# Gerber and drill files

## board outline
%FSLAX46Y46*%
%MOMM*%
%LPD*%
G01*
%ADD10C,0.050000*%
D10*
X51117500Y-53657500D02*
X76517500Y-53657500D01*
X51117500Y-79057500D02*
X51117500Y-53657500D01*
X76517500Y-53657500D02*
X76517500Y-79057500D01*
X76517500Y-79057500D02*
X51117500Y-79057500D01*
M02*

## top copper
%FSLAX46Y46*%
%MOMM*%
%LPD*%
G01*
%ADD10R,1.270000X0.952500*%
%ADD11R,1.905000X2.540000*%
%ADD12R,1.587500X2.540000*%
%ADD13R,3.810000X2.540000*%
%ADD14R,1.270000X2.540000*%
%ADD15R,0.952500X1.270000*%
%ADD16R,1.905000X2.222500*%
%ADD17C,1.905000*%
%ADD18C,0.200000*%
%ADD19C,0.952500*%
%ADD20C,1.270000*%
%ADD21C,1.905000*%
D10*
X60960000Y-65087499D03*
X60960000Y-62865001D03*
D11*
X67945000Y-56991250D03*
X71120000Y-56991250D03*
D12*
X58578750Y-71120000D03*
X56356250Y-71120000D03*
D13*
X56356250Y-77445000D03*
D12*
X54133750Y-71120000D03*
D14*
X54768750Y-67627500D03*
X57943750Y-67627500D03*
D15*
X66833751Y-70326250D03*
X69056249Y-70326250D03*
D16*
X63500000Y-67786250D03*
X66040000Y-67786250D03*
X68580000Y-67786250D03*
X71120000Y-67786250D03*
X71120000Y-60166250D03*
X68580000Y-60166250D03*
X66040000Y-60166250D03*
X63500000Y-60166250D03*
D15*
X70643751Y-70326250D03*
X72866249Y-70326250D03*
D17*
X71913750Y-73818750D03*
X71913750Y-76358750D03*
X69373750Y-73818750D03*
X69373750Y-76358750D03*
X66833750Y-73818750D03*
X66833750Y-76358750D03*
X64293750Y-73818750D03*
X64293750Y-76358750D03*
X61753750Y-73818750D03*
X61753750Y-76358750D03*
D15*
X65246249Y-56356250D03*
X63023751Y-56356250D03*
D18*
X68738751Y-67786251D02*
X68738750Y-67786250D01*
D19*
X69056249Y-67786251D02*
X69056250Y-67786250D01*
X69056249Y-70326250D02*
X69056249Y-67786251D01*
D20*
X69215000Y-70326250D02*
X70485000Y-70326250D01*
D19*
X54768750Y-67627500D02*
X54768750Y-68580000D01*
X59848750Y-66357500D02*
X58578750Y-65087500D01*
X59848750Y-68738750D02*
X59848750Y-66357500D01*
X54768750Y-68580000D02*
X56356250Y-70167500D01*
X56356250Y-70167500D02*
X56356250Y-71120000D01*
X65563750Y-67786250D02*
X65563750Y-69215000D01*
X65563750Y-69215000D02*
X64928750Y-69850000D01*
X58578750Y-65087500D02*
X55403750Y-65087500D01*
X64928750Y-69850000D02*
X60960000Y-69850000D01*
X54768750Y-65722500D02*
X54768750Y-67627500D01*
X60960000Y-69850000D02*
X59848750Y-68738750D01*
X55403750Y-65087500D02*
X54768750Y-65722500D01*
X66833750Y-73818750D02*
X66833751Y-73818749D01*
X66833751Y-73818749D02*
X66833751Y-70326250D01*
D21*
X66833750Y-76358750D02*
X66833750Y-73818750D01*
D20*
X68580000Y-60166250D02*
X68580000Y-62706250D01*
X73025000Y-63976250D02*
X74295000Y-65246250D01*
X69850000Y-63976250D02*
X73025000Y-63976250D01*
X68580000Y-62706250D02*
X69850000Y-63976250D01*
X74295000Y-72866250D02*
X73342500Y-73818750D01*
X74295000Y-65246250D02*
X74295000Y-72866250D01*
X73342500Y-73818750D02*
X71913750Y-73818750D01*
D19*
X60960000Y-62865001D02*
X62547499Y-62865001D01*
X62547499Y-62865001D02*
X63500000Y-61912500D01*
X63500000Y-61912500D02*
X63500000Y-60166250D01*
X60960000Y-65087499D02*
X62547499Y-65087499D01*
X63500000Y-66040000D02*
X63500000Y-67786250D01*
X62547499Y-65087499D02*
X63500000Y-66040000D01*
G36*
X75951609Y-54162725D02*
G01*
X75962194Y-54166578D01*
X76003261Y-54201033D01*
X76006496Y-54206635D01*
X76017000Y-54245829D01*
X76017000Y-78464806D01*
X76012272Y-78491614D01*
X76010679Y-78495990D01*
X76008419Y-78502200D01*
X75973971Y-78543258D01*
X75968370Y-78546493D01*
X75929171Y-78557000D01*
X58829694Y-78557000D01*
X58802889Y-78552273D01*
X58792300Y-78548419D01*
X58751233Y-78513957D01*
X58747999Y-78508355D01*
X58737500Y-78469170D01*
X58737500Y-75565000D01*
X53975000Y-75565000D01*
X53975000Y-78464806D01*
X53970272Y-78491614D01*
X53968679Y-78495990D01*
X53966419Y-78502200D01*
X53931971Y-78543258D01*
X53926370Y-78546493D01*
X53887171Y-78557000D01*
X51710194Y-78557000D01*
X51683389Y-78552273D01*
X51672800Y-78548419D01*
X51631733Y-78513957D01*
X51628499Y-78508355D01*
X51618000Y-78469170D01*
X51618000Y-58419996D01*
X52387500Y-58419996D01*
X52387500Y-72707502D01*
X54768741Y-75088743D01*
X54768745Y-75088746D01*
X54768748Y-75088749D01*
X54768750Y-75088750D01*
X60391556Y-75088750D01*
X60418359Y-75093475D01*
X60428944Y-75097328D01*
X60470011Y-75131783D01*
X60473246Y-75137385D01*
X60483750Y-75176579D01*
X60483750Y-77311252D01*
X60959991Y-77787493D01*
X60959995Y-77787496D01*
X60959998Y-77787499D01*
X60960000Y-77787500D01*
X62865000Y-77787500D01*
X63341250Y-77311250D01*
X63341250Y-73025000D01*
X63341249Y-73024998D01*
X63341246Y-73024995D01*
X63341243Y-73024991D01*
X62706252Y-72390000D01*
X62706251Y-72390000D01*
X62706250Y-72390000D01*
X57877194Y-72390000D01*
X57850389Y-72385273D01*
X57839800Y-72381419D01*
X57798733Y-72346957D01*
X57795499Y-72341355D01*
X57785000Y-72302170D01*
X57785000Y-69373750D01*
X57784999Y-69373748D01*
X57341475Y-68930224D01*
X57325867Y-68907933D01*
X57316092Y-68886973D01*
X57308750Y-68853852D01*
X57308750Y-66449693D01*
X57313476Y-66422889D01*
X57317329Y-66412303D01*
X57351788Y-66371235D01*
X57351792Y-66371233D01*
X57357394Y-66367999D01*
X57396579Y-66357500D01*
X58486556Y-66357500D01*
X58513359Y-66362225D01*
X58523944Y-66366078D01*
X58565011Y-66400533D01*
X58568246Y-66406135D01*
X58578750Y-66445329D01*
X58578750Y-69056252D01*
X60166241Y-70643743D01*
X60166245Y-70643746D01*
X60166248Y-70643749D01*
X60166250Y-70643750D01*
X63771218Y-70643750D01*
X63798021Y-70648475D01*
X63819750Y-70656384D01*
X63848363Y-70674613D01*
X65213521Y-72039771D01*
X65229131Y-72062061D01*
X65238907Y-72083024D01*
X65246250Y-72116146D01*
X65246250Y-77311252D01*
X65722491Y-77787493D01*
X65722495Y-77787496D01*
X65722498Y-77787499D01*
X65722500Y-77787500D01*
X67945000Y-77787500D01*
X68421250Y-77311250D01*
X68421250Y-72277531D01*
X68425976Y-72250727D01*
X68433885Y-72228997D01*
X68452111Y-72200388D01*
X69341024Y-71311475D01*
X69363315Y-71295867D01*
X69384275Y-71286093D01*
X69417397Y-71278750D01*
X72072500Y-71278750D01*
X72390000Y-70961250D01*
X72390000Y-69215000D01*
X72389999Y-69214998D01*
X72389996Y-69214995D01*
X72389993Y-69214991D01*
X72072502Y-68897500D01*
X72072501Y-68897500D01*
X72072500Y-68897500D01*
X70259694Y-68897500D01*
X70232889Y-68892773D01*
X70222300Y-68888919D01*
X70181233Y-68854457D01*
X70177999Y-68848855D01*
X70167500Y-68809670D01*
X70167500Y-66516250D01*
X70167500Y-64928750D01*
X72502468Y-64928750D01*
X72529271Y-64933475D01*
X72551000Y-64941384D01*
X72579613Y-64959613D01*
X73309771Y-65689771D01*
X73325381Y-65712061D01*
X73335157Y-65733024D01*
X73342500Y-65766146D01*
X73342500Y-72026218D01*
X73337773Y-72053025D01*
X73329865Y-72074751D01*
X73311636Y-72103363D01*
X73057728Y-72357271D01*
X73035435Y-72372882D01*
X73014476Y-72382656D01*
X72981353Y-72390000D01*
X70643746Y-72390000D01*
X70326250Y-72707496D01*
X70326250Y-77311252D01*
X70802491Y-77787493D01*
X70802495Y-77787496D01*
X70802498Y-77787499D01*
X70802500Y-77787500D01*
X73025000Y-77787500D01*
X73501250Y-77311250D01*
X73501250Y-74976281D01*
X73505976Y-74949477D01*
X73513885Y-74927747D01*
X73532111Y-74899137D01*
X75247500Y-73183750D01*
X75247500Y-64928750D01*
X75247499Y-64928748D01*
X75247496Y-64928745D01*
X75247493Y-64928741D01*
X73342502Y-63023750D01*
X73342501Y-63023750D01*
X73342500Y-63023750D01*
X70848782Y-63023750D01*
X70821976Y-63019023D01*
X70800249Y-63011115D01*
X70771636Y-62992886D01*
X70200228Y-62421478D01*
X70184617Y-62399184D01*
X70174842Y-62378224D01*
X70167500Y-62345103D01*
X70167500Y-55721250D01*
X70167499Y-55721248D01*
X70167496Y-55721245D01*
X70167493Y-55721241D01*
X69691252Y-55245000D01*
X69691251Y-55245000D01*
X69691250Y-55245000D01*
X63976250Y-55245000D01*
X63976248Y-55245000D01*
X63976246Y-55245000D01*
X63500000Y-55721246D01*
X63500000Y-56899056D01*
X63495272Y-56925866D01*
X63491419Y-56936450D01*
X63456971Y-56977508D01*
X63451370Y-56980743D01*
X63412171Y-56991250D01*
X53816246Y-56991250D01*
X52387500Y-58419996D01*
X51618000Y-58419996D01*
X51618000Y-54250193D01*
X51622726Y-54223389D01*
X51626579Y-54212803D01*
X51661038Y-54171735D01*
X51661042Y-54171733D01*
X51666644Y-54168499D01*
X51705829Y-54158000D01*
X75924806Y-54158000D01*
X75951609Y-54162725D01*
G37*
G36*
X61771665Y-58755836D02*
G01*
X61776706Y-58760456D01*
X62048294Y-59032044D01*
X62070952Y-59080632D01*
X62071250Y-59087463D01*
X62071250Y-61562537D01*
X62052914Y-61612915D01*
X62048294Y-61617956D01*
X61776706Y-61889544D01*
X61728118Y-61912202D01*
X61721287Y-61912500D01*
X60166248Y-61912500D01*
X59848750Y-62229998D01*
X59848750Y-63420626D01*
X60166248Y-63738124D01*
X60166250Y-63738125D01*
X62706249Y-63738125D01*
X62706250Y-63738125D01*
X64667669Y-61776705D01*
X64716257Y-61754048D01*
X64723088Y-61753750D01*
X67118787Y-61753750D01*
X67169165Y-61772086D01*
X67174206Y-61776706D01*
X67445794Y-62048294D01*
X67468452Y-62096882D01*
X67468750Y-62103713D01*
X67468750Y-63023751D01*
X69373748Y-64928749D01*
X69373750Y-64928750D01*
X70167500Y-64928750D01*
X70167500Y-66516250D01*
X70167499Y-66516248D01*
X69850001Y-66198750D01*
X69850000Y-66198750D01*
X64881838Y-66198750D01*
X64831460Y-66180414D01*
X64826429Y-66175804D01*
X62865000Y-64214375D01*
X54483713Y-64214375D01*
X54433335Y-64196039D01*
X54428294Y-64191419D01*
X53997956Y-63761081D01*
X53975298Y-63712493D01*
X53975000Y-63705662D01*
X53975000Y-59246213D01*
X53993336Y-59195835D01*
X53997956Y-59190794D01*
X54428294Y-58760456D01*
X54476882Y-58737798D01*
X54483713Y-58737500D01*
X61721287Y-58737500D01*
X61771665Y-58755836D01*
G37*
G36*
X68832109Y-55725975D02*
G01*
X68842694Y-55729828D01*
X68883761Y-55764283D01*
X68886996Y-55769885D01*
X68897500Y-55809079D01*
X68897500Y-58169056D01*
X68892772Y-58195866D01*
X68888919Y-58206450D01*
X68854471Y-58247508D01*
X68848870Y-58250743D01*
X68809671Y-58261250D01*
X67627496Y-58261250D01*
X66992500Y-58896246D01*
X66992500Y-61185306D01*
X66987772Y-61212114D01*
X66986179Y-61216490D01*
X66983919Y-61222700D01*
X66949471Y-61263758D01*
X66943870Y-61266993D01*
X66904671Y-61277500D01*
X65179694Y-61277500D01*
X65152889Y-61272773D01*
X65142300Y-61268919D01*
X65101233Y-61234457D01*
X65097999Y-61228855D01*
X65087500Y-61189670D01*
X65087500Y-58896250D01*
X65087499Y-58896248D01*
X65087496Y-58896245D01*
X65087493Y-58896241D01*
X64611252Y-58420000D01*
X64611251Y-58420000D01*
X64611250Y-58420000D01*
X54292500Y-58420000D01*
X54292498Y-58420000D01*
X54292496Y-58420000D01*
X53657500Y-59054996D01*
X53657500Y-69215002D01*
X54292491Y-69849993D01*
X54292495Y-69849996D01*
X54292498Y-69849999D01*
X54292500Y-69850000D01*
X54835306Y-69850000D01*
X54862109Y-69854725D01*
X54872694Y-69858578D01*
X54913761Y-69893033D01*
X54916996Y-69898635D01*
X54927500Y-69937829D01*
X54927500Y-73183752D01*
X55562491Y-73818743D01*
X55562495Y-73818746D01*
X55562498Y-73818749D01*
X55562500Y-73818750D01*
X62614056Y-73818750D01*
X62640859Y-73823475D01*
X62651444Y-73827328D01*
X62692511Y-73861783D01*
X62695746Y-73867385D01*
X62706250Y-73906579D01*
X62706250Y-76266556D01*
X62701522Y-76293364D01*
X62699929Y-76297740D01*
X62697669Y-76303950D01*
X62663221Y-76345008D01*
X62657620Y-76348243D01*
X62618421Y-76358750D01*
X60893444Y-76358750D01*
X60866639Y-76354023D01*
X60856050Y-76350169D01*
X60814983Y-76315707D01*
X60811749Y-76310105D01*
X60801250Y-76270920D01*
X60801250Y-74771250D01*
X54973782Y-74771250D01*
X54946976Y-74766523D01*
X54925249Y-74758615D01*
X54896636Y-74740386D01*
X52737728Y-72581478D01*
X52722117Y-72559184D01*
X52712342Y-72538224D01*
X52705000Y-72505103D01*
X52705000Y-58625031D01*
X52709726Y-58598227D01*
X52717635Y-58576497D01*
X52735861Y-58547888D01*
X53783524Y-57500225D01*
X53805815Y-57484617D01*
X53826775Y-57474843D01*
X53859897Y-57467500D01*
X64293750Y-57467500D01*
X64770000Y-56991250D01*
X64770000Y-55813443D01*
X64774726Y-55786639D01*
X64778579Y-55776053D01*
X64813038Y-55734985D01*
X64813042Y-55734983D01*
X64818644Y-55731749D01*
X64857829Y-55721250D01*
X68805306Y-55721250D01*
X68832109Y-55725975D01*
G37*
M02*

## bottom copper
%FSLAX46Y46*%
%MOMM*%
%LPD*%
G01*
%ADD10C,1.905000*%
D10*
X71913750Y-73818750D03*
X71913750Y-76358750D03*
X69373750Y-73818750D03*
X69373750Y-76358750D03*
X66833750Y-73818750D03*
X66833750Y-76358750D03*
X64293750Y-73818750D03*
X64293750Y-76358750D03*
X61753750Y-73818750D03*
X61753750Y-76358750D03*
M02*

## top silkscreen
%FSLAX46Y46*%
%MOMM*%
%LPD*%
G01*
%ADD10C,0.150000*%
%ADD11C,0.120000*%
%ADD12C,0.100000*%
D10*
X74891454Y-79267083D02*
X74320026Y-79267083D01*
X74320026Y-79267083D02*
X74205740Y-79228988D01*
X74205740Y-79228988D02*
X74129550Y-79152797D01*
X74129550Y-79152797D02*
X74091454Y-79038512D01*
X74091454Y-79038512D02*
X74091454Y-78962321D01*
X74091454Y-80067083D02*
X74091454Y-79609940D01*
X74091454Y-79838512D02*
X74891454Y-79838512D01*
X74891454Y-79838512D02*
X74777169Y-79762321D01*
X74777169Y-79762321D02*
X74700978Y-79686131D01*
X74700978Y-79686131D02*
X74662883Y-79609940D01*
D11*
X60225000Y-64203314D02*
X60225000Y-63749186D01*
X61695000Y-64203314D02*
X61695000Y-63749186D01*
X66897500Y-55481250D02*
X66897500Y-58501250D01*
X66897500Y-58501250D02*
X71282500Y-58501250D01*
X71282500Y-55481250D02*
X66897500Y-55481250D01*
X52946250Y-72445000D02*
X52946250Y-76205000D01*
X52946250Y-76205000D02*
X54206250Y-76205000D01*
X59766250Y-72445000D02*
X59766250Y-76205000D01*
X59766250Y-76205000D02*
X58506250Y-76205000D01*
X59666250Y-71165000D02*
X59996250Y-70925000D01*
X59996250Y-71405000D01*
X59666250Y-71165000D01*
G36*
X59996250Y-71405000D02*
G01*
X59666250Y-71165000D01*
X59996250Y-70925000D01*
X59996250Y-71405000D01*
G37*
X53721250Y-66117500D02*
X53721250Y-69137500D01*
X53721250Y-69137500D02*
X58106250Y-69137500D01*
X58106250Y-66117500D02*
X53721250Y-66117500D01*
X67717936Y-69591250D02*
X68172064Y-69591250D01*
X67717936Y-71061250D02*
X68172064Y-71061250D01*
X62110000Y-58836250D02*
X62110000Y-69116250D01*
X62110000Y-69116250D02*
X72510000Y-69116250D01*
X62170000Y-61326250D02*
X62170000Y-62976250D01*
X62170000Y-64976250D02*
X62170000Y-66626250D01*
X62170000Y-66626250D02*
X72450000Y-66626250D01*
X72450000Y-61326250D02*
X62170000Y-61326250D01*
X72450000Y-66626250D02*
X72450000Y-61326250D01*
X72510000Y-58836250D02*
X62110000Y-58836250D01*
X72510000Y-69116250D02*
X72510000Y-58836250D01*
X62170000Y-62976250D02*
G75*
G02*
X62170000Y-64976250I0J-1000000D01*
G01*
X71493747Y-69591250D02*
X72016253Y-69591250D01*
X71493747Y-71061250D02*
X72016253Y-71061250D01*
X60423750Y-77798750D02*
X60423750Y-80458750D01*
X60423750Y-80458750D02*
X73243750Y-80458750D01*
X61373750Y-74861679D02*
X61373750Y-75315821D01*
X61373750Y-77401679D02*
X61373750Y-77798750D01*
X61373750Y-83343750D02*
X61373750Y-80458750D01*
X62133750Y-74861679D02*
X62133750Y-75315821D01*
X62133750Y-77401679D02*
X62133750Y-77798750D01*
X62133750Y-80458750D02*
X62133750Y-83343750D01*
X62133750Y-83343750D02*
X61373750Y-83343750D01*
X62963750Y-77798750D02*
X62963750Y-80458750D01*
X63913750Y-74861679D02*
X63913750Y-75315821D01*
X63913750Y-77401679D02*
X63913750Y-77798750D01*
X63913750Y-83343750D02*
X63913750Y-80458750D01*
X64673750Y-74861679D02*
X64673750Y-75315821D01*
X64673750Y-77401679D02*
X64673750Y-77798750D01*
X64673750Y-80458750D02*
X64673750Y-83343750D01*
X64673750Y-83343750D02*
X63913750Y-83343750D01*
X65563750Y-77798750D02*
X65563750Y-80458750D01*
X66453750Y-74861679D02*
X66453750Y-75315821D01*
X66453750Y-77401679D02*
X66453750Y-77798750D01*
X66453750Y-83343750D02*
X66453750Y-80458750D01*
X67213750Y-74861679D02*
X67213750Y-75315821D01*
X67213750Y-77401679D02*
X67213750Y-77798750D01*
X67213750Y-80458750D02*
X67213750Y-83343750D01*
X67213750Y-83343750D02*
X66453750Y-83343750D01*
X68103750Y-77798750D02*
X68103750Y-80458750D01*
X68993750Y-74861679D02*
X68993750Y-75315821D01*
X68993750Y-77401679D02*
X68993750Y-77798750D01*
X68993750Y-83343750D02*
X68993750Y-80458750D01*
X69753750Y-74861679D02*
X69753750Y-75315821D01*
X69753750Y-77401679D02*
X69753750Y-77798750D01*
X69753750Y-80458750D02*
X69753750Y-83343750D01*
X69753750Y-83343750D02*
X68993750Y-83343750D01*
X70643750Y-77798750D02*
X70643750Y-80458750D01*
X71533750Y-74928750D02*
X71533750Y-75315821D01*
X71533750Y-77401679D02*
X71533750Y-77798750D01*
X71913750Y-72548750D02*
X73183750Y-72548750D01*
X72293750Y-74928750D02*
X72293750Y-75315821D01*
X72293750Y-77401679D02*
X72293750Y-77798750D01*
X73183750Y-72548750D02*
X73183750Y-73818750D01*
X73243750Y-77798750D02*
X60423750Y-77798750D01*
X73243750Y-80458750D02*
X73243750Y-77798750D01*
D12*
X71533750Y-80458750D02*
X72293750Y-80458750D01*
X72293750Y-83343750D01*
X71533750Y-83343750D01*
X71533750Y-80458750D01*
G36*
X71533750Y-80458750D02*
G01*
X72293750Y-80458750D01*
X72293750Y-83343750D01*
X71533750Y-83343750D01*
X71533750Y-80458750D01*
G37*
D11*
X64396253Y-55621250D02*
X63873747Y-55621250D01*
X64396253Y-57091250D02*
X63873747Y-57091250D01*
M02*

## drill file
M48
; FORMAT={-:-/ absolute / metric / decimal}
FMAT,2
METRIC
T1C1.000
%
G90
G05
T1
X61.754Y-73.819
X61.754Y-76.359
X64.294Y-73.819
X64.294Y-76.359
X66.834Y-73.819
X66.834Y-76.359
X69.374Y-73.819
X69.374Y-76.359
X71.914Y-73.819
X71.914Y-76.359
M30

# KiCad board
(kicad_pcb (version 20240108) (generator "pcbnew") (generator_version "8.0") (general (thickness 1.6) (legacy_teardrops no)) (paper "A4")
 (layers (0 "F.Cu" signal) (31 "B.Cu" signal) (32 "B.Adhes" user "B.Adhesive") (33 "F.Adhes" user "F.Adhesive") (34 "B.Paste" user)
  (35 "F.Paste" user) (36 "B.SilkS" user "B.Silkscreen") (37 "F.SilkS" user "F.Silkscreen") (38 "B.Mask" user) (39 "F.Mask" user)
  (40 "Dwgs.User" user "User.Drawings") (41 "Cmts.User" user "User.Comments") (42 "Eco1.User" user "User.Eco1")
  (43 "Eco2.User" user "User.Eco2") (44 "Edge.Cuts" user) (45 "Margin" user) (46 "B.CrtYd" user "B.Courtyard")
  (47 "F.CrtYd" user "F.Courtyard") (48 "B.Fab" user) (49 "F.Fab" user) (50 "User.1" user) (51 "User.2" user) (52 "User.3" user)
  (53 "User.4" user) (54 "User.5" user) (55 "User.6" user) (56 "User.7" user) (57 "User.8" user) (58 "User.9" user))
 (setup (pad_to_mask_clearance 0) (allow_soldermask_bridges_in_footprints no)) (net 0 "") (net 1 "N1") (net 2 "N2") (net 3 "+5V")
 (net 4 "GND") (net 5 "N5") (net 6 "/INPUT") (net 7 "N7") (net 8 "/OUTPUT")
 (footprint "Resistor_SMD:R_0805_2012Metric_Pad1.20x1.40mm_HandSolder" (layer "F.Cu") (at 60.96 63.97625 90)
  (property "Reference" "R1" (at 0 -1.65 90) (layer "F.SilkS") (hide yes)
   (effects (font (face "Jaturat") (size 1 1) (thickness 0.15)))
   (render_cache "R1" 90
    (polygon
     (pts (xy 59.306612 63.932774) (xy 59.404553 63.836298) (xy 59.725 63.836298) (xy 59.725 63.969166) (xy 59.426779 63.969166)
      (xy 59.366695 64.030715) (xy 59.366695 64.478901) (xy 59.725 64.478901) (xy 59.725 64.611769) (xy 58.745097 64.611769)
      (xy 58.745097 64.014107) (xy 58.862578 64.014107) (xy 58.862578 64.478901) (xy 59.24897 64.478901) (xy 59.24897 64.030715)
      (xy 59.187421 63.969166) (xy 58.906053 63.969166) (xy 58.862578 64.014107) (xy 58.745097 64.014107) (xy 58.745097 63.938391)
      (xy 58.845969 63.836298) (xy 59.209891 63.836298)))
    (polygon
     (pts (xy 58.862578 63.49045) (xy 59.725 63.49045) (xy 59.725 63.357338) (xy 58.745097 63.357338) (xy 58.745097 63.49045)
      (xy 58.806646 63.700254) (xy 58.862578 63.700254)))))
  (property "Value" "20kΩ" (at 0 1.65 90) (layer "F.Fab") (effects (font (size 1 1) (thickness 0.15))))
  (fp_line (start -0.227064 -0.735) (end 0.227064 -0.735) (stroke (width 0.12) (type solid)) (layer "F.SilkS"))
  (fp_line (start -0.227064 0.735) (end 0.227064 0.735) (stroke (width 0.12) (type solid)) (layer "F.SilkS"))
  (pad "1" smd rect (at -1.111249 0 90) (size 0.9525 1.27) (layers "F.Cu" "F.Paste" "F.Mask") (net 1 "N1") (clearance 0.15875))
  (pad "2" smd rect (at 1.111249 0 90) (size 0.9525 1.27) (layers "F.Cu" "F.Paste" "F.Mask") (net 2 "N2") (clearance 0.15875)))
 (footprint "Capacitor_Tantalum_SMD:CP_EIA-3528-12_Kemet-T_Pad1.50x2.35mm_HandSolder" (layer "F.Cu") (at 69.5325 56.99125)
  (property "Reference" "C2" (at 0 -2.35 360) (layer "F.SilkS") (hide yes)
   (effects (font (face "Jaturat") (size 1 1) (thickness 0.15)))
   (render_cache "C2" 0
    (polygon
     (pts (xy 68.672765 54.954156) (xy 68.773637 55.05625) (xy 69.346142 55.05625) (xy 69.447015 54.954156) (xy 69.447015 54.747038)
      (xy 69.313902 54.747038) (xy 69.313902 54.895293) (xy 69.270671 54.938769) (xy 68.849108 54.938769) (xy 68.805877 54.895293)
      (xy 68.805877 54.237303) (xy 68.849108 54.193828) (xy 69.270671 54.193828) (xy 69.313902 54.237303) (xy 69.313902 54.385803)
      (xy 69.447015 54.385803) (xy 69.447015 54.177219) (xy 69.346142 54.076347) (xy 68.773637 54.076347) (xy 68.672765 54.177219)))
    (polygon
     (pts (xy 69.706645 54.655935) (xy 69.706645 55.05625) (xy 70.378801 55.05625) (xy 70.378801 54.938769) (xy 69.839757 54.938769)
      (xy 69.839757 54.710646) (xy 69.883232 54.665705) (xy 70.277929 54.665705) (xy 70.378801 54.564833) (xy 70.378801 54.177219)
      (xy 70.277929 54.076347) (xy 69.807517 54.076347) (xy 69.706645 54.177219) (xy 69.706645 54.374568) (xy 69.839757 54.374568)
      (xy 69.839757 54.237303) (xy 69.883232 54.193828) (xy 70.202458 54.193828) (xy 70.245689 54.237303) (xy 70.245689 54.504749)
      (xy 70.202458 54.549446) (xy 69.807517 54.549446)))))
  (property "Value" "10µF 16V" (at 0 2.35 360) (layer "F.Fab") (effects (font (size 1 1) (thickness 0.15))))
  (fp_line (start -2.635 -1.51) (end -2.635 1.51) (stroke (width 0.12) (type solid)) (layer "F.SilkS"))
  (fp_line (start -2.635 1.51) (end 1.75 1.51) (stroke (width 0.12) (type solid)) (layer "F.SilkS"))
  (fp_line (start 1.75 -1.51) (end -2.635 -1.51) (stroke (width 0.12) (type solid)) (layer "F.SilkS"))
  (pad "1" smd rect (at -1.5875 0) (size 1.905 2.54) (layers "F.Cu" "F.Paste" "F.Mask") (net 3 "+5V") (clearance 0.15875))
  (pad "2" smd rect (at 1.5875 0) (size 1.905 2.54) (layers "F.Cu" "F.Paste" "F.Mask") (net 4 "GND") (clearance 0.15875)))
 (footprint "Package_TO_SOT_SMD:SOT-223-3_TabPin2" (layer "F.Cu") (at 56.35625 74.295 -90)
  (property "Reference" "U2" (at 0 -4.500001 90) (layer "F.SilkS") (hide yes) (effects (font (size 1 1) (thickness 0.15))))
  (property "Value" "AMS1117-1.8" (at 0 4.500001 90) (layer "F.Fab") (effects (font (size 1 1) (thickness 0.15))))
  (fp_line (start -1.85 3.41) (end 1.91 3.41) (stroke (width 0.12) (type solid)) (layer "F.SilkS"))
  (fp_line (start 1.91 3.41) (end 1.91 2.15) (stroke (width 0.12) (type solid)) (layer "F.SilkS"))
  (fp_line (start -1.85 -3.41) (end 1.91 -3.41) (stroke (width 0.12) (type solid)) (layer "F.SilkS"))
  (fp_line (start 1.91 -3.41) (end 1.91 -2.15) (stroke (width 0.12) (type solid)) (layer "F.SilkS"))
  (fp_poly
   (pts (xy -3.13 -3.31) (xy -3.37 -3.64) (xy -2.89 -3.64) (xy -3.13 -3.31)) (stroke (width 0.12) (type solid)) (fill solid)
   (layer "F.SilkS"))
  (pad "1" smd rect (at -3.175 -2.2225 270) (size 2.54 1.5875) (layers "F.Cu" "F.Paste" "F.Mask") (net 4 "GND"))
  (pad "2" smd rect (at -3.175 0 270) (size 2.54 1.5875) (layers "F.Cu" "F.Paste" "F.Mask") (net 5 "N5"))
  (pad "2" smd rect (at 3.15 0 270) (size 2.54 3.81) (layers "F.Cu" "F.Paste" "F.Mask") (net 5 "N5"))
  (pad "3" smd rect (at -3.175 2.2225 270) (size 2.54 1.5875) (layers "F.Cu" "F.Paste" "F.Mask") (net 3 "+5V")))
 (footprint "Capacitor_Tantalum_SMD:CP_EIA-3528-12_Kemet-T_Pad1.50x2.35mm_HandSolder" (layer "F.Cu") (at 56.35625 67.6275)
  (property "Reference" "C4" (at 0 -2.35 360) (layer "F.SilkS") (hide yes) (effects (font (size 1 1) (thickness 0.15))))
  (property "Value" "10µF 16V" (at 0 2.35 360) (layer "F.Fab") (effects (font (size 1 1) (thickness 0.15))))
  (fp_line (start -2.635 -1.51) (end -2.635 1.51) (stroke (width 0.12) (type solid)) (layer "F.SilkS"))
  (fp_line (start -2.635 1.51) (end 1.75 1.51) (stroke (width 0.12) (type solid)) (layer "F.SilkS"))
  (fp_line (start 1.75 -1.51) (end -2.635 -1.51) (stroke (width 0.12) (type solid)) (layer "F.SilkS"))
  (pad "1" smd rect (at -1.5875 0) (size 1.27 2.54) (layers "F.Cu" "F.Paste" "F.Mask") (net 5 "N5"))
  (pad "2" smd rect (at 1.5875 0) (size 1.27 2.54) (layers "F.Cu" "F.Paste" "F.Mask") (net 4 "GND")))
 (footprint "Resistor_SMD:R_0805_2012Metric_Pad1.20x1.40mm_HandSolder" (layer "F.Cu") (at 67.945 70.32625)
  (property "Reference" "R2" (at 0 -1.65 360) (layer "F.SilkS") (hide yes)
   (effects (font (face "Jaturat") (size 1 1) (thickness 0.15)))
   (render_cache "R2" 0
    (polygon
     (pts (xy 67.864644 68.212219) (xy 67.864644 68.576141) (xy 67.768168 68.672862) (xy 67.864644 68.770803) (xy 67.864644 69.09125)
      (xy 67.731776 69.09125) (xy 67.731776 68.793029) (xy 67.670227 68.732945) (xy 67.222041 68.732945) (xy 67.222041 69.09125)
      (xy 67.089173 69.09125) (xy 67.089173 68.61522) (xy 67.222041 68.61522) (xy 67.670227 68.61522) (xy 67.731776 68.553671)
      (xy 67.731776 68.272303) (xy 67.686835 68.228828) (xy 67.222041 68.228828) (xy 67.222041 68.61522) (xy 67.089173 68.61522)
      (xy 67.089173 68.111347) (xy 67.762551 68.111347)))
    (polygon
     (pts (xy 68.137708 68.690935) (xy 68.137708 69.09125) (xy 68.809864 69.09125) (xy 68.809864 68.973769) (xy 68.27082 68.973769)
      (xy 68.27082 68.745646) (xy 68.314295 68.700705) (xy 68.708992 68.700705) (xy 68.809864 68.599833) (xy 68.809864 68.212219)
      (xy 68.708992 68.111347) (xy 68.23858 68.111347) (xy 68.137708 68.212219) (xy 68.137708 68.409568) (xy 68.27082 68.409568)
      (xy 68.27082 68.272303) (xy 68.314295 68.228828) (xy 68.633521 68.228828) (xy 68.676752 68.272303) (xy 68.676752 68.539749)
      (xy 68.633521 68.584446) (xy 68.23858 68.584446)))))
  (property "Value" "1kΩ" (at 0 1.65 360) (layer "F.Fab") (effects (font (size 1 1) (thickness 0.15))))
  (fp_line (start -0.227064 -0.735) (end 0.227064 -0.735) (stroke (width 0.12) (type solid)) (layer "F.SilkS"))
  (fp_line (start -0.227064 0.735) (end 0.227064 0.735) (stroke (width 0.12) (type solid)) (layer "F.SilkS"))
  (pad "1" smd rect (at -1.111249 0) (size 0.9525 1.27) (layers "F.Cu" "F.Paste" "F.Mask") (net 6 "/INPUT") (clearance 0.15875))
  (pad "2" smd rect (at 1.111249 0) (size 0.9525 1.27) (layers "F.Cu" "F.Paste" "F.Mask") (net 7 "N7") (clearance 0.15875)))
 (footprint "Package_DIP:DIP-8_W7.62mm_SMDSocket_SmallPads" (layer "F.Cu") (at 67.31 63.97625 90)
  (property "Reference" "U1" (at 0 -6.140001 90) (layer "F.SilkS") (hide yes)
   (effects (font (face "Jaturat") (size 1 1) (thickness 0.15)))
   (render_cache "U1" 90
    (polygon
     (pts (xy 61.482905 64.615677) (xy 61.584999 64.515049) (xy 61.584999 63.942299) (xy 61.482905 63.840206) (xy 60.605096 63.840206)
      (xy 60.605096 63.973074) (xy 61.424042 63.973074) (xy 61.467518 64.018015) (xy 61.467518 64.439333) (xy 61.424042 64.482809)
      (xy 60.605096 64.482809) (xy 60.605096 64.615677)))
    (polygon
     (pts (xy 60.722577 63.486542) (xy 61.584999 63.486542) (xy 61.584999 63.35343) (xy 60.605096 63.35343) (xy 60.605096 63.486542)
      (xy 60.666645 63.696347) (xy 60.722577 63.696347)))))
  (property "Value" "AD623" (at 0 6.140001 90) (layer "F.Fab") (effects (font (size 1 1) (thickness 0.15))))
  (fp_line (start 5.14 -5.2) (end -5.14 -5.2) (stroke (width 0.12) (type solid)) (layer "F.SilkS"))
  (fp_line (start -5.14 -5.2) (end -5.14 5.2) (stroke (width 0.12) (type solid)) (layer "F.SilkS"))
  (fp_line (start 2.65 -5.14) (end 1 -5.14) (stroke (width 0.12) (type solid)) (layer "F.SilkS"))
  (fp_line (start -1 -5.14) (end -2.65 -5.14) (stroke (width 0.12) (type solid)) (layer "F.SilkS"))
  (fp_line (start -2.65 -5.14) (end -2.65 5.14) (stroke (width 0.12) (type solid)) (layer "F.SilkS"))
  (fp_line (start 2.65 5.14) (end 2.65 -5.14) (stroke (width 0.12) (type solid)) (layer "F.SilkS"))
  (fp_line (start -2.65 5.14) (end 2.65 5.14) (stroke (width 0.12) (type solid)) (layer "F.SilkS"))
  (fp_line (start 5.14 5.2) (end 5.14 -5.2) (stroke (width 0.12) (type solid)) (layer "F.SilkS"))
  (fp_line (start -5.14 5.2) (end 5.14 5.2) (stroke (width 0.12) (type solid)) (layer "F.SilkS"))
  (fp_arc (start 1 -5.14) (mid 0 -4.14) (end -1 -5.14) (stroke (width 0.12) (type solid)) (layer "F.SilkS"))
  (pad "1" smd rect (at -3.81 -3.81 90) (size 2.2225 1.905) (layers "F.Cu" "F.Paste" "F.Mask") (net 1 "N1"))
  (pad "2" smd rect (at -3.81 -1.27 90) (size 2.2225 1.905) (layers "F.Cu" "F.Paste" "F.Mask") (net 5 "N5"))
  (pad "3" smd rect (at -3.81 1.27 90) (size 2.2225 1.905) (layers "F.Cu" "F.Paste" "F.Mask") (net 7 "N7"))
  (pad "4" smd rect (at -3.81 3.81 90) (size 2.2225 1.905) (layers "F.Cu" "F.Paste" "F.Mask") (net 4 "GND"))
  (pad "5" smd rect (at 3.81 3.81 90) (size 2.2225 1.905) (layers "F.Cu" "F.Paste" "F.Mask") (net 4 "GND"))
  (pad "6" smd rect (at 3.81 1.27 90) (size 2.2225 1.905) (layers "F.Cu" "F.Paste" "F.Mask") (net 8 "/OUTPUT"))
  (pad "7" smd rect (at 3.81 -1.27 90) (size 2.2225 1.905) (layers "F.Cu" "F.Paste" "F.Mask") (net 3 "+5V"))
  (pad "8" smd rect (at 3.81 -3.81 90) (size 2.2225 1.905) (layers "F.Cu" "F.Paste" "F.Mask") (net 2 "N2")))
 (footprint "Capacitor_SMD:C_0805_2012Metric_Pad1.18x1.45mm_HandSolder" (layer "F.Cu") (at 71.755 70.32625)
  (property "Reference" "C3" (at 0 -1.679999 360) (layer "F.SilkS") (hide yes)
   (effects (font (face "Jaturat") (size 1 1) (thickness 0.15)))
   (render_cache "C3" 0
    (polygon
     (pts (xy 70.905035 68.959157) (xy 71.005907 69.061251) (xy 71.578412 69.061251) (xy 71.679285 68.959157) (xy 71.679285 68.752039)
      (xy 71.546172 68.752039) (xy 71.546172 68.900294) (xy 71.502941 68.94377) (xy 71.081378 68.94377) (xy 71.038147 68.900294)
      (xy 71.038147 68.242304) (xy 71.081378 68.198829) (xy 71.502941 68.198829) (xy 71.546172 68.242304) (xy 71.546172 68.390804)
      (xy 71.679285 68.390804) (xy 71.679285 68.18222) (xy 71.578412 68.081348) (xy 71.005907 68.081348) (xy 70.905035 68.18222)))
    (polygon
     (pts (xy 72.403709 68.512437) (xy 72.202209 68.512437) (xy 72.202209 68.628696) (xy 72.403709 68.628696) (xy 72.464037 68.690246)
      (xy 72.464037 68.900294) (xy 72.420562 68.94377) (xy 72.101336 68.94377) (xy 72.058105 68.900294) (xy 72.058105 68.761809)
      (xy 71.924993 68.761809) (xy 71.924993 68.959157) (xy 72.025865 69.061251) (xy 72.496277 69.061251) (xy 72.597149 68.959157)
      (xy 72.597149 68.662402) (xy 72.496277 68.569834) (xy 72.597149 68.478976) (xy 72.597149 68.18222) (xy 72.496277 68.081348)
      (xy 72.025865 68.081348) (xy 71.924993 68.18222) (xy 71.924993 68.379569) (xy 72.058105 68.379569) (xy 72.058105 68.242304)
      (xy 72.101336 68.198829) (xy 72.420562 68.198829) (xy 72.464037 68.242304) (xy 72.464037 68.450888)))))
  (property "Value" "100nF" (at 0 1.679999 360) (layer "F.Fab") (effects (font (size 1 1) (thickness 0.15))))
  (fp_line (start -0.261253 -0.735) (end 0.261253 -0.735) (stroke (width 0.12) (type solid)) (layer "F.SilkS"))
  (fp_line (start -0.261253 0.735) (end 0.261253 0.735) (stroke (width 0.12) (type solid)) (layer "F.SilkS"))
  (pad "1" smd rect (at -1.111249 0) (size 0.9525 1.27) (layers "F.Cu" "F.Paste" "F.Mask") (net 7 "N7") (clearance 0.15875))
  (pad "2" smd rect (at 1.111249 0) (size 0.9525 1.27) (layers "F.Cu" "F.Paste" "F.Mask") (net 4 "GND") (clearance 0.15875)))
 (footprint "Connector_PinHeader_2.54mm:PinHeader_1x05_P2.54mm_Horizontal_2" (layer "F.Cu") (at 71.91375 73.81875 -90)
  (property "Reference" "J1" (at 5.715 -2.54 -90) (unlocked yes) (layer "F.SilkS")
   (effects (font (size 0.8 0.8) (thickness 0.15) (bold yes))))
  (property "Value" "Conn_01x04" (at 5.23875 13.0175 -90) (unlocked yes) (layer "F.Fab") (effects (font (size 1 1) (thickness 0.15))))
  (fp_line (start 3.98 11.49) (end 6.64 11.49) (stroke (width 0.12) (type solid)) (layer "F.SilkS"))
  (fp_line (start 6.64 11.49) (end 6.64 -1.33) (stroke (width 0.12) (type solid)) (layer "F.SilkS"))
  (fp_line (start 1.042929 10.54) (end 1.497071 10.54) (stroke (width 0.12) (type solid)) (layer "F.SilkS"))
  (fp_line (start 3.582929 10.54) (end 3.98 10.54) (stroke (width 0.12) (type solid)) (layer "F.SilkS"))
  (fp_line (start 9.525 10.54) (end 6.64 10.54) (stroke (width 0.12) (type solid)) (layer "F.SilkS"))
  (fp_line (start 1.042929 9.78) (end 1.497071 9.78) (stroke (width 0.12) (type solid)) (layer "F.SilkS"))
  (fp_line (start 3.582929 9.78) (end 3.98 9.78) (stroke (width 0.12) (type solid)) (layer "F.SilkS"))
  (fp_line (start 6.64 9.78) (end 9.525 9.78) (stroke (width 0.12) (type solid)) (layer "F.SilkS"))
  (fp_line (start 9.525 9.78) (end 9.525 10.54) (stroke (width 0.12) (type solid)) (layer "F.SilkS"))
  (fp_line (start 3.98 8.95) (end 6.64 8.95) (stroke (width 0.12) (type solid)) (layer "F.SilkS"))
  (fp_line (start 1.042929 8) (end 1.497071 8) (stroke (width 0.12) (type solid)) (layer "F.SilkS"))
  (fp_line (start 3.582929 8) (end 3.98 8) (stroke (width 0.12) (type solid)) (layer "F.SilkS"))
  (fp_line (start 9.525 8) (end 6.64 8) (stroke (width 0.12) (type solid)) (layer "F.SilkS"))
  (fp_line (start 1.042929 7.24) (end 1.497071 7.24) (stroke (width 0.12) (type solid)) (layer "F.SilkS"))
  (fp_line (start 3.582929 7.24) (end 3.98 7.24) (stroke (width 0.12) (type solid)) (layer "F.SilkS"))
  (fp_line (start 6.64 7.24) (end 9.525 7.24) (stroke (width 0.12) (type solid)) (layer "F.SilkS"))
  (fp_line (start 9.525 7.24) (end 9.525 8) (stroke (width 0.12) (type solid)) (layer "F.SilkS"))
  (fp_line (start 3.98 6.35) (end 6.64 6.35) (stroke (width 0.12) (type solid)) (layer "F.SilkS"))
  (fp_line (start 1.042929 5.46) (end 1.497071 5.46) (stroke (width 0.12) (type solid)) (layer "F.SilkS"))
  (fp_line (start 3.582929 5.46) (end 3.98 5.46) (stroke (width 0.12) (type solid)) (layer "F.SilkS"))
  (fp_line (start 9.525 5.46) (end 6.64 5.46) (stroke (width 0.12) (type solid)) (layer "F.SilkS"))
  (fp_line (start 1.042929 4.7) (end 1.497071 4.7) (stroke (width 0.12) (type solid)) (layer "F.SilkS"))
  (fp_line (start 3.582929 4.7) (end 3.98 4.7) (stroke (width 0.12) (type solid)) (layer "F.SilkS"))
  (fp_line (start 6.64 4.7) (end 9.525 4.7) (stroke (width 0.12) (type solid)) (layer "F.SilkS"))
  (fp_line (start 9.525 4.7) (end 9.525 5.46) (stroke (width 0.12) (type solid)) (layer "F.SilkS"))
  (fp_line (start 3.98 3.81) (end 6.64 3.81) (stroke (width 0.12) (type solid)) (layer "F.SilkS"))
  (fp_line (start 1.042929 2.92) (end 1.497071 2.92) (stroke (width 0.12) (type solid)) (layer "F.SilkS"))
  (fp_line (start 3.582929 2.92) (end 3.98 2.92) (stroke (width 0.12) (type solid)) (layer "F.SilkS"))
  (fp_line (start 9.525 2.92) (end 6.64 2.92) (stroke (width 0.12) (type solid)) (layer "F.SilkS"))
  (fp_line (start 1.042929 2.16) (end 1.497071 2.16) (stroke (width 0.12) (type solid)) (layer "F.SilkS"))
  (fp_line (start 3.582929 2.16) (end 3.98 2.16) (stroke (width 0.12) (type solid)) (layer "F.SilkS"))
  (fp_line (start 6.64 2.16) (end 9.525 2.16) (stroke (width 0.12) (type solid)) (layer "F.SilkS"))
  (fp_line (start 9.525 2.16) (end 9.525 2.92) (stroke (width 0.12) (type solid)) (layer "F.SilkS"))
  (fp_line (start 3.98 1.27) (end 6.64 1.27) (stroke (width 0.12) (type solid)) (layer "F.SilkS"))
  (fp_line (start 1.11 0.38) (end 1.497071 0.38) (stroke (width 0.12) (type solid)) (layer "F.SilkS"))
  (fp_line (start 3.582929 0.38) (end 3.98 0.38) (stroke (width 0.12) (type solid)) (layer "F.SilkS"))
  (fp_line (start -1.27 0) (end -1.27 -1.27) (stroke (width 0.12) (type solid)) (layer "F.SilkS"))
  (fp_line (start 1.11 -0.38) (end 1.497071 -0.38) (stroke (width 0.12) (type solid)) (layer "F.SilkS"))
  (fp_line (start 3.582929 -0.38) (end 3.98 -0.38) (stroke (width 0.12) (type solid)) (layer "F.SilkS"))
  (fp_line (start -1.27 -1.27) (end 0 -1.27) (stroke (width 0.12) (type solid)) (layer "F.SilkS"))
  (fp_line (start 3.98 -1.33) (end 3.98 11.49) (stroke (width 0.12) (type solid)) (layer "F.SilkS"))
  (fp_line (start 6.64 -1.33) (end 3.98 -1.33) (stroke (width 0.12) (type solid)) (layer "F.SilkS"))
  (fp_rect (start 6.64 -0.38) (end 9.525 0.38) (stroke (width 0.1) (type solid)) (fill solid) (layer "F.SilkS"))
  (pad "1" thru_hole circle (at 0 0 270) (size 1.905 1.905) (drill 1) (layers "*.Cu" "*.Mask") (remove_unused_layers no) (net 8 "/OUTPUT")
   (thermal_bridge_angle 90))
  (pad "1" thru_hole circle (at 2.54 0 270) (size 1.905 1.905) (drill 1) (layers "*.Cu" "*.Mask") (remove_unused_layers no)
   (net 8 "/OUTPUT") (thermal_bridge_angle 90))
  (pad "2" thru_hole circle (at 0 2.54 270) (size 1.905 1.905) (drill 1) (layers "*.Cu" "*.Mask") (remove_unused_layers no) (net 4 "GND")
   (thermal_bridge_angle 90))
  (pad "2" thru_hole circle (at 2.54 2.54 270) (size 1.905 1.905) (drill 1) (layers "*.Cu" "*.Mask") (remove_unused_layers no) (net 4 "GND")
   (thermal_bridge_angle 90))
  (pad "3" thru_hole circle (at 0 5.08 270) (size 1.905 1.905) (drill 1) (layers "*.Cu" "*.Mask") (remove_unused_layers no) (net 6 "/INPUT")
   (thermal_bridge_angle 90))
  (pad "3" thru_hole circle (at 2.54 5.08 270) (size 1.905 1.905) (drill 1) (layers "*.Cu" "*.Mask") (remove_unused_layers no)
   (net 6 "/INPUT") (thermal_bridge_angle 90))
  (pad "4" thru_hole circle (at 0 7.62 270) (size 1.905 1.905) (drill 1) (layers "*.Cu" "*.Mask") (remove_unused_layers no) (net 4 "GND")
   (thermal_bridge_angle 90))
  (pad "4" thru_hole circle (at 2.54 7.62 270) (size 1.905 1.905) (drill 1) (layers "*.Cu" "*.Mask") (remove_unused_layers no) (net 4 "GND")
   (thermal_bridge_angle 90))
  (pad "5" thru_hole circle (at 0 10.16 270) (size 1.905 1.905) (drill 1) (layers "*.Cu" "*.Mask") (remove_unused_layers no) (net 3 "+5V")
   (thermal_bridge_angle 90))
  (pad "5" thru_hole circle (at 2.54 10.16 270) (size 1.905 1.905) (drill 1) (layers "*.Cu" "*.Mask") (remove_unused_layers no)
   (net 3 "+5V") (thermal_bridge_angle 90)))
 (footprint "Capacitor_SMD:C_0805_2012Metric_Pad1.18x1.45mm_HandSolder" (layer "F.Cu") (at 64.135 56.35625 180)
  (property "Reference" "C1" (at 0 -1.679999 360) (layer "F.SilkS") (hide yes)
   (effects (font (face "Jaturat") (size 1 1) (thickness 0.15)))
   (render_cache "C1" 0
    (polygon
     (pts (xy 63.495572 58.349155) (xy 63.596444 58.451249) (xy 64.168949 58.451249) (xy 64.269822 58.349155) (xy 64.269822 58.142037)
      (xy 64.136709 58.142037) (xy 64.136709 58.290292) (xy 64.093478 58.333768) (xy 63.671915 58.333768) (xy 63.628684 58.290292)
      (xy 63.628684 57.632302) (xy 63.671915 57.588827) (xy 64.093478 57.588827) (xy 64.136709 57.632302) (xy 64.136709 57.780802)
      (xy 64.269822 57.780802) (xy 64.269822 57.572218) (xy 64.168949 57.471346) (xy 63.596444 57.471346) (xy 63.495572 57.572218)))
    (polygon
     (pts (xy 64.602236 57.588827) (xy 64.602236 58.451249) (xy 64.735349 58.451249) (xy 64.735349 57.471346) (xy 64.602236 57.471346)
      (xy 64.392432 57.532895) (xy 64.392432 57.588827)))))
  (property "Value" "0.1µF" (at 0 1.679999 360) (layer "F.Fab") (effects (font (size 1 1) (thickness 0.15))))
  (fp_line (start -0.261253 0.735) (end 0.261253 0.735) (stroke (width 0.12) (type solid)) (layer "F.SilkS"))
  (fp_line (start -0.261253 -0.735) (end 0.261253 -0.735) (stroke (width 0.12) (type solid)) (layer "F.SilkS"))
  (pad "1" smd rect (at -1.111249 0 180) (size 0.9525 1.27) (layers "F.Cu" "F.Paste" "F.Mask") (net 3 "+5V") (clearance 0.15875))
  (pad "2" smd rect (at 1.111249 0 180) (size 0.9525 1.27) (layers "F.Cu" "F.Paste" "F.Mask") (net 4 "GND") (clearance 0.15875)))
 (gr_line (start 51.1175 53.6575) (end 76.5175 53.6575) (stroke (width 0.05) (type default)) (layer "Edge.Cuts"))
 (gr_line (start 51.1175 79.0575) (end 51.1175 53.6575) (stroke (width 0.05) (type default)) (layer "Edge.Cuts"))
 (gr_line (start 76.5175 53.6575) (end 76.5175 79.0575) (stroke (width 0.05) (type default)) (layer "Edge.Cuts"))
 (gr_line (start 76.5175 79.0575) (end 51.1175 79.0575) (stroke (width 0.05) (type default)) (layer "Edge.Cuts"))
 (segment (start 68.738751 67.786251) (end 68.73875 67.78625) (width 0.2) (layer "F.Cu") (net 7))
 (segment (start 69.056249 67.786251) (end 69.05625 67.78625) (width 0.9525) (layer "F.Cu") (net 7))
 (segment (start 69.056249 70.32625) (end 69.056249 67.786251) (width 0.9525) (layer "F.Cu") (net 7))
 (segment (start 69.215 70.32625) (end 70.485 70.32625) (width 1.27) (layer "F.Cu") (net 7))
 (segment (start 54.76875 67.6275) (end 54.76875 68.58) (width 0.9525) (layer "F.Cu") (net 5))
 (segment (start 59.84875 66.3575) (end 58.57875 65.0875) (width 0.9525) (layer "F.Cu") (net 5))
 (segment (start 59.84875 68.73875) (end 59.84875 66.3575) (width 0.9525) (layer "F.Cu") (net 5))
 (segment (start 54.76875 68.58) (end 56.35625 70.1675) (width 0.9525) (layer "F.Cu") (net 5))
 (segment (start 56.35625 70.1675) (end 56.35625 71.12) (width 0.9525) (layer "F.Cu") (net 5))
 (segment (start 65.56375 67.78625) (end 65.56375 69.215) (width 0.9525) (layer "F.Cu") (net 5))
 (segment (start 65.56375 69.215) (end 64.92875 69.85) (width 0.9525) (layer "F.Cu") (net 5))
 (segment (start 58.57875 65.0875) (end 55.40375 65.0875) (width 0.9525) (layer "F.Cu") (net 5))
 (segment (start 64.92875 69.85) (end 60.96 69.85) (width 0.9525) (layer "F.Cu") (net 5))
 (segment (start 54.76875 65.7225) (end 54.76875 67.6275) (width 0.9525) (layer "F.Cu") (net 5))
 (segment (start 60.96 69.85) (end 59.84875 68.73875) (width 0.9525) (layer "F.Cu") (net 5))
 (segment (start 55.40375 65.0875) (end 54.76875 65.7225) (width 0.9525) (layer "F.Cu") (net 5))
 (segment (start 66.83375 73.81875) (end 66.833751 73.818749) (width 0.9525) (layer "F.Cu") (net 6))
 (segment (start 66.833751 73.818749) (end 66.833751 70.32625) (width 0.9525) (layer "F.Cu") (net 6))
 (segment (start 66.83375 76.35875) (end 66.83375 73.81875) (width 1.905) (layer "F.Cu") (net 6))
 (segment (start 68.58 60.16625) (end 68.58 62.70625) (width 1.27) (layer "F.Cu") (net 8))
 (segment (start 73.025 63.97625) (end 74.295 65.24625) (width 1.27) (layer "F.Cu") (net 8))
 (segment (start 69.85 63.97625) (end 73.025 63.97625) (width 1.27) (layer "F.Cu") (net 8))
 (segment (start 68.58 62.70625) (end 69.85 63.97625) (width 1.27) (layer "F.Cu") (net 8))
 (segment (start 74.295 72.86625) (end 73.3425 73.81875) (width 1.27) (layer "F.Cu") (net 8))
 (segment (start 74.295 65.24625) (end 74.295 72.86625) (width 1.27) (layer "F.Cu") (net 8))
 (segment (start 73.3425 73.81875) (end 71.91375 73.81875) (width 1.27) (layer "F.Cu") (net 8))
 (segment (start 60.96 62.865001) (end 62.547499 62.865001) (width 0.9525) (layer "F.Cu") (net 2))
 (segment (start 62.547499 62.865001) (end 63.5 61.9125) (width 0.9525) (layer "F.Cu") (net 2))
 (segment (start 63.5 61.9125) (end 63.5 60.16625) (width 0.9525) (layer "F.Cu") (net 2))
 (segment (start 60.96 65.087499) (end 62.547499 65.087499) (width 0.9525) (layer "F.Cu") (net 1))
 (segment (start 63.5 66.04) (end 63.5 67.78625) (width 0.9525) (layer "F.Cu") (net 1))
 (segment (start 62.547499 65.087499) (end 63.5 66.04) (width 0.9525) (layer "F.Cu") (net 1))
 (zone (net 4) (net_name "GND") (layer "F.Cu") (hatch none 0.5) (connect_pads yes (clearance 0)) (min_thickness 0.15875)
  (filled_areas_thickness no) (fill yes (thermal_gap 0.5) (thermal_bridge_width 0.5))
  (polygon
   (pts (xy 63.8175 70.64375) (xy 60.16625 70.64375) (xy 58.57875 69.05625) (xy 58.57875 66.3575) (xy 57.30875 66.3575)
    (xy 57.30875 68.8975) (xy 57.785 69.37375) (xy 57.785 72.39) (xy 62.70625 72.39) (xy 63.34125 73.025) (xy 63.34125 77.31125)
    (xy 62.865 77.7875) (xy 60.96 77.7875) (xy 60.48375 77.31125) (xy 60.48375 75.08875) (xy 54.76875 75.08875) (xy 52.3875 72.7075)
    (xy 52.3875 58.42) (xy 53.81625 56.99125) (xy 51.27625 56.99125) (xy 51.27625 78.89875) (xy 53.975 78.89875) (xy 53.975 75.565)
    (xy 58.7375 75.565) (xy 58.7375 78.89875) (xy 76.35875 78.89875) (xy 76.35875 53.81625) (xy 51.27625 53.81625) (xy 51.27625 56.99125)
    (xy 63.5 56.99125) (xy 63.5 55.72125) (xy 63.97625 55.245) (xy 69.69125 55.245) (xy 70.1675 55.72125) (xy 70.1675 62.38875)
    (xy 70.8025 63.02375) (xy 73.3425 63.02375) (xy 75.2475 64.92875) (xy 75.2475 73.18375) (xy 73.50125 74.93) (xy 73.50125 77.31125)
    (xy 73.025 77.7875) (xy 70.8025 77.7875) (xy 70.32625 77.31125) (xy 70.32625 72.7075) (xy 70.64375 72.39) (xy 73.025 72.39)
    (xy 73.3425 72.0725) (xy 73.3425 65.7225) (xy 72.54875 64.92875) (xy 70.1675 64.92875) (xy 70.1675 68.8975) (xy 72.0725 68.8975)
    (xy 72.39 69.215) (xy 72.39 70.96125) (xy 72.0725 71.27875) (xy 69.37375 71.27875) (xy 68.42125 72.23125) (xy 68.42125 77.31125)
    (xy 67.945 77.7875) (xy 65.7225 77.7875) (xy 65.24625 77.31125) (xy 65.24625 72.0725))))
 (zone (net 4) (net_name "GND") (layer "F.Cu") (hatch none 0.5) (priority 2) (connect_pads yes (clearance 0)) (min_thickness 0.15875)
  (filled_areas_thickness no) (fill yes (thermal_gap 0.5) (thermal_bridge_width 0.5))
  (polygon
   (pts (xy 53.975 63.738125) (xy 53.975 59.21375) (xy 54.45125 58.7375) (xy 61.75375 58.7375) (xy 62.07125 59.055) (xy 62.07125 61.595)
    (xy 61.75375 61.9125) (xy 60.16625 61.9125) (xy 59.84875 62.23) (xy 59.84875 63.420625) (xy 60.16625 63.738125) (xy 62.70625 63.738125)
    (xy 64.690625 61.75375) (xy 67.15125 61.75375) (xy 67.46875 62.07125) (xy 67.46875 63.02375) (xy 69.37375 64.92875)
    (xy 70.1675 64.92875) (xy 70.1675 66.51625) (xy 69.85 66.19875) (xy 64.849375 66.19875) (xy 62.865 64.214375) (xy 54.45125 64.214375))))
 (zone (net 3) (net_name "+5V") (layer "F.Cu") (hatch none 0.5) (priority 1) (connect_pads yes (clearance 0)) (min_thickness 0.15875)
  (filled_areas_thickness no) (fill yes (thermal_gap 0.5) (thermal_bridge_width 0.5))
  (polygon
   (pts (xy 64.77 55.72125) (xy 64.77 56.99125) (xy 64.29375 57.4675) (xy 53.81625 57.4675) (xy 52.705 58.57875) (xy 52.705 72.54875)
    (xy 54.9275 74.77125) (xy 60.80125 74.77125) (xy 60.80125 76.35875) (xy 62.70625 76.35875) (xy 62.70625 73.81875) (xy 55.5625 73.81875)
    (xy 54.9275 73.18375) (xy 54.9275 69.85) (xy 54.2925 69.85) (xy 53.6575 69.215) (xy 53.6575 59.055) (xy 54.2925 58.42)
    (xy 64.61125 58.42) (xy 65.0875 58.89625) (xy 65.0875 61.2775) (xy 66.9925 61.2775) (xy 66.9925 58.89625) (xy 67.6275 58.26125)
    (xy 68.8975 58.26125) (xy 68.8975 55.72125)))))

